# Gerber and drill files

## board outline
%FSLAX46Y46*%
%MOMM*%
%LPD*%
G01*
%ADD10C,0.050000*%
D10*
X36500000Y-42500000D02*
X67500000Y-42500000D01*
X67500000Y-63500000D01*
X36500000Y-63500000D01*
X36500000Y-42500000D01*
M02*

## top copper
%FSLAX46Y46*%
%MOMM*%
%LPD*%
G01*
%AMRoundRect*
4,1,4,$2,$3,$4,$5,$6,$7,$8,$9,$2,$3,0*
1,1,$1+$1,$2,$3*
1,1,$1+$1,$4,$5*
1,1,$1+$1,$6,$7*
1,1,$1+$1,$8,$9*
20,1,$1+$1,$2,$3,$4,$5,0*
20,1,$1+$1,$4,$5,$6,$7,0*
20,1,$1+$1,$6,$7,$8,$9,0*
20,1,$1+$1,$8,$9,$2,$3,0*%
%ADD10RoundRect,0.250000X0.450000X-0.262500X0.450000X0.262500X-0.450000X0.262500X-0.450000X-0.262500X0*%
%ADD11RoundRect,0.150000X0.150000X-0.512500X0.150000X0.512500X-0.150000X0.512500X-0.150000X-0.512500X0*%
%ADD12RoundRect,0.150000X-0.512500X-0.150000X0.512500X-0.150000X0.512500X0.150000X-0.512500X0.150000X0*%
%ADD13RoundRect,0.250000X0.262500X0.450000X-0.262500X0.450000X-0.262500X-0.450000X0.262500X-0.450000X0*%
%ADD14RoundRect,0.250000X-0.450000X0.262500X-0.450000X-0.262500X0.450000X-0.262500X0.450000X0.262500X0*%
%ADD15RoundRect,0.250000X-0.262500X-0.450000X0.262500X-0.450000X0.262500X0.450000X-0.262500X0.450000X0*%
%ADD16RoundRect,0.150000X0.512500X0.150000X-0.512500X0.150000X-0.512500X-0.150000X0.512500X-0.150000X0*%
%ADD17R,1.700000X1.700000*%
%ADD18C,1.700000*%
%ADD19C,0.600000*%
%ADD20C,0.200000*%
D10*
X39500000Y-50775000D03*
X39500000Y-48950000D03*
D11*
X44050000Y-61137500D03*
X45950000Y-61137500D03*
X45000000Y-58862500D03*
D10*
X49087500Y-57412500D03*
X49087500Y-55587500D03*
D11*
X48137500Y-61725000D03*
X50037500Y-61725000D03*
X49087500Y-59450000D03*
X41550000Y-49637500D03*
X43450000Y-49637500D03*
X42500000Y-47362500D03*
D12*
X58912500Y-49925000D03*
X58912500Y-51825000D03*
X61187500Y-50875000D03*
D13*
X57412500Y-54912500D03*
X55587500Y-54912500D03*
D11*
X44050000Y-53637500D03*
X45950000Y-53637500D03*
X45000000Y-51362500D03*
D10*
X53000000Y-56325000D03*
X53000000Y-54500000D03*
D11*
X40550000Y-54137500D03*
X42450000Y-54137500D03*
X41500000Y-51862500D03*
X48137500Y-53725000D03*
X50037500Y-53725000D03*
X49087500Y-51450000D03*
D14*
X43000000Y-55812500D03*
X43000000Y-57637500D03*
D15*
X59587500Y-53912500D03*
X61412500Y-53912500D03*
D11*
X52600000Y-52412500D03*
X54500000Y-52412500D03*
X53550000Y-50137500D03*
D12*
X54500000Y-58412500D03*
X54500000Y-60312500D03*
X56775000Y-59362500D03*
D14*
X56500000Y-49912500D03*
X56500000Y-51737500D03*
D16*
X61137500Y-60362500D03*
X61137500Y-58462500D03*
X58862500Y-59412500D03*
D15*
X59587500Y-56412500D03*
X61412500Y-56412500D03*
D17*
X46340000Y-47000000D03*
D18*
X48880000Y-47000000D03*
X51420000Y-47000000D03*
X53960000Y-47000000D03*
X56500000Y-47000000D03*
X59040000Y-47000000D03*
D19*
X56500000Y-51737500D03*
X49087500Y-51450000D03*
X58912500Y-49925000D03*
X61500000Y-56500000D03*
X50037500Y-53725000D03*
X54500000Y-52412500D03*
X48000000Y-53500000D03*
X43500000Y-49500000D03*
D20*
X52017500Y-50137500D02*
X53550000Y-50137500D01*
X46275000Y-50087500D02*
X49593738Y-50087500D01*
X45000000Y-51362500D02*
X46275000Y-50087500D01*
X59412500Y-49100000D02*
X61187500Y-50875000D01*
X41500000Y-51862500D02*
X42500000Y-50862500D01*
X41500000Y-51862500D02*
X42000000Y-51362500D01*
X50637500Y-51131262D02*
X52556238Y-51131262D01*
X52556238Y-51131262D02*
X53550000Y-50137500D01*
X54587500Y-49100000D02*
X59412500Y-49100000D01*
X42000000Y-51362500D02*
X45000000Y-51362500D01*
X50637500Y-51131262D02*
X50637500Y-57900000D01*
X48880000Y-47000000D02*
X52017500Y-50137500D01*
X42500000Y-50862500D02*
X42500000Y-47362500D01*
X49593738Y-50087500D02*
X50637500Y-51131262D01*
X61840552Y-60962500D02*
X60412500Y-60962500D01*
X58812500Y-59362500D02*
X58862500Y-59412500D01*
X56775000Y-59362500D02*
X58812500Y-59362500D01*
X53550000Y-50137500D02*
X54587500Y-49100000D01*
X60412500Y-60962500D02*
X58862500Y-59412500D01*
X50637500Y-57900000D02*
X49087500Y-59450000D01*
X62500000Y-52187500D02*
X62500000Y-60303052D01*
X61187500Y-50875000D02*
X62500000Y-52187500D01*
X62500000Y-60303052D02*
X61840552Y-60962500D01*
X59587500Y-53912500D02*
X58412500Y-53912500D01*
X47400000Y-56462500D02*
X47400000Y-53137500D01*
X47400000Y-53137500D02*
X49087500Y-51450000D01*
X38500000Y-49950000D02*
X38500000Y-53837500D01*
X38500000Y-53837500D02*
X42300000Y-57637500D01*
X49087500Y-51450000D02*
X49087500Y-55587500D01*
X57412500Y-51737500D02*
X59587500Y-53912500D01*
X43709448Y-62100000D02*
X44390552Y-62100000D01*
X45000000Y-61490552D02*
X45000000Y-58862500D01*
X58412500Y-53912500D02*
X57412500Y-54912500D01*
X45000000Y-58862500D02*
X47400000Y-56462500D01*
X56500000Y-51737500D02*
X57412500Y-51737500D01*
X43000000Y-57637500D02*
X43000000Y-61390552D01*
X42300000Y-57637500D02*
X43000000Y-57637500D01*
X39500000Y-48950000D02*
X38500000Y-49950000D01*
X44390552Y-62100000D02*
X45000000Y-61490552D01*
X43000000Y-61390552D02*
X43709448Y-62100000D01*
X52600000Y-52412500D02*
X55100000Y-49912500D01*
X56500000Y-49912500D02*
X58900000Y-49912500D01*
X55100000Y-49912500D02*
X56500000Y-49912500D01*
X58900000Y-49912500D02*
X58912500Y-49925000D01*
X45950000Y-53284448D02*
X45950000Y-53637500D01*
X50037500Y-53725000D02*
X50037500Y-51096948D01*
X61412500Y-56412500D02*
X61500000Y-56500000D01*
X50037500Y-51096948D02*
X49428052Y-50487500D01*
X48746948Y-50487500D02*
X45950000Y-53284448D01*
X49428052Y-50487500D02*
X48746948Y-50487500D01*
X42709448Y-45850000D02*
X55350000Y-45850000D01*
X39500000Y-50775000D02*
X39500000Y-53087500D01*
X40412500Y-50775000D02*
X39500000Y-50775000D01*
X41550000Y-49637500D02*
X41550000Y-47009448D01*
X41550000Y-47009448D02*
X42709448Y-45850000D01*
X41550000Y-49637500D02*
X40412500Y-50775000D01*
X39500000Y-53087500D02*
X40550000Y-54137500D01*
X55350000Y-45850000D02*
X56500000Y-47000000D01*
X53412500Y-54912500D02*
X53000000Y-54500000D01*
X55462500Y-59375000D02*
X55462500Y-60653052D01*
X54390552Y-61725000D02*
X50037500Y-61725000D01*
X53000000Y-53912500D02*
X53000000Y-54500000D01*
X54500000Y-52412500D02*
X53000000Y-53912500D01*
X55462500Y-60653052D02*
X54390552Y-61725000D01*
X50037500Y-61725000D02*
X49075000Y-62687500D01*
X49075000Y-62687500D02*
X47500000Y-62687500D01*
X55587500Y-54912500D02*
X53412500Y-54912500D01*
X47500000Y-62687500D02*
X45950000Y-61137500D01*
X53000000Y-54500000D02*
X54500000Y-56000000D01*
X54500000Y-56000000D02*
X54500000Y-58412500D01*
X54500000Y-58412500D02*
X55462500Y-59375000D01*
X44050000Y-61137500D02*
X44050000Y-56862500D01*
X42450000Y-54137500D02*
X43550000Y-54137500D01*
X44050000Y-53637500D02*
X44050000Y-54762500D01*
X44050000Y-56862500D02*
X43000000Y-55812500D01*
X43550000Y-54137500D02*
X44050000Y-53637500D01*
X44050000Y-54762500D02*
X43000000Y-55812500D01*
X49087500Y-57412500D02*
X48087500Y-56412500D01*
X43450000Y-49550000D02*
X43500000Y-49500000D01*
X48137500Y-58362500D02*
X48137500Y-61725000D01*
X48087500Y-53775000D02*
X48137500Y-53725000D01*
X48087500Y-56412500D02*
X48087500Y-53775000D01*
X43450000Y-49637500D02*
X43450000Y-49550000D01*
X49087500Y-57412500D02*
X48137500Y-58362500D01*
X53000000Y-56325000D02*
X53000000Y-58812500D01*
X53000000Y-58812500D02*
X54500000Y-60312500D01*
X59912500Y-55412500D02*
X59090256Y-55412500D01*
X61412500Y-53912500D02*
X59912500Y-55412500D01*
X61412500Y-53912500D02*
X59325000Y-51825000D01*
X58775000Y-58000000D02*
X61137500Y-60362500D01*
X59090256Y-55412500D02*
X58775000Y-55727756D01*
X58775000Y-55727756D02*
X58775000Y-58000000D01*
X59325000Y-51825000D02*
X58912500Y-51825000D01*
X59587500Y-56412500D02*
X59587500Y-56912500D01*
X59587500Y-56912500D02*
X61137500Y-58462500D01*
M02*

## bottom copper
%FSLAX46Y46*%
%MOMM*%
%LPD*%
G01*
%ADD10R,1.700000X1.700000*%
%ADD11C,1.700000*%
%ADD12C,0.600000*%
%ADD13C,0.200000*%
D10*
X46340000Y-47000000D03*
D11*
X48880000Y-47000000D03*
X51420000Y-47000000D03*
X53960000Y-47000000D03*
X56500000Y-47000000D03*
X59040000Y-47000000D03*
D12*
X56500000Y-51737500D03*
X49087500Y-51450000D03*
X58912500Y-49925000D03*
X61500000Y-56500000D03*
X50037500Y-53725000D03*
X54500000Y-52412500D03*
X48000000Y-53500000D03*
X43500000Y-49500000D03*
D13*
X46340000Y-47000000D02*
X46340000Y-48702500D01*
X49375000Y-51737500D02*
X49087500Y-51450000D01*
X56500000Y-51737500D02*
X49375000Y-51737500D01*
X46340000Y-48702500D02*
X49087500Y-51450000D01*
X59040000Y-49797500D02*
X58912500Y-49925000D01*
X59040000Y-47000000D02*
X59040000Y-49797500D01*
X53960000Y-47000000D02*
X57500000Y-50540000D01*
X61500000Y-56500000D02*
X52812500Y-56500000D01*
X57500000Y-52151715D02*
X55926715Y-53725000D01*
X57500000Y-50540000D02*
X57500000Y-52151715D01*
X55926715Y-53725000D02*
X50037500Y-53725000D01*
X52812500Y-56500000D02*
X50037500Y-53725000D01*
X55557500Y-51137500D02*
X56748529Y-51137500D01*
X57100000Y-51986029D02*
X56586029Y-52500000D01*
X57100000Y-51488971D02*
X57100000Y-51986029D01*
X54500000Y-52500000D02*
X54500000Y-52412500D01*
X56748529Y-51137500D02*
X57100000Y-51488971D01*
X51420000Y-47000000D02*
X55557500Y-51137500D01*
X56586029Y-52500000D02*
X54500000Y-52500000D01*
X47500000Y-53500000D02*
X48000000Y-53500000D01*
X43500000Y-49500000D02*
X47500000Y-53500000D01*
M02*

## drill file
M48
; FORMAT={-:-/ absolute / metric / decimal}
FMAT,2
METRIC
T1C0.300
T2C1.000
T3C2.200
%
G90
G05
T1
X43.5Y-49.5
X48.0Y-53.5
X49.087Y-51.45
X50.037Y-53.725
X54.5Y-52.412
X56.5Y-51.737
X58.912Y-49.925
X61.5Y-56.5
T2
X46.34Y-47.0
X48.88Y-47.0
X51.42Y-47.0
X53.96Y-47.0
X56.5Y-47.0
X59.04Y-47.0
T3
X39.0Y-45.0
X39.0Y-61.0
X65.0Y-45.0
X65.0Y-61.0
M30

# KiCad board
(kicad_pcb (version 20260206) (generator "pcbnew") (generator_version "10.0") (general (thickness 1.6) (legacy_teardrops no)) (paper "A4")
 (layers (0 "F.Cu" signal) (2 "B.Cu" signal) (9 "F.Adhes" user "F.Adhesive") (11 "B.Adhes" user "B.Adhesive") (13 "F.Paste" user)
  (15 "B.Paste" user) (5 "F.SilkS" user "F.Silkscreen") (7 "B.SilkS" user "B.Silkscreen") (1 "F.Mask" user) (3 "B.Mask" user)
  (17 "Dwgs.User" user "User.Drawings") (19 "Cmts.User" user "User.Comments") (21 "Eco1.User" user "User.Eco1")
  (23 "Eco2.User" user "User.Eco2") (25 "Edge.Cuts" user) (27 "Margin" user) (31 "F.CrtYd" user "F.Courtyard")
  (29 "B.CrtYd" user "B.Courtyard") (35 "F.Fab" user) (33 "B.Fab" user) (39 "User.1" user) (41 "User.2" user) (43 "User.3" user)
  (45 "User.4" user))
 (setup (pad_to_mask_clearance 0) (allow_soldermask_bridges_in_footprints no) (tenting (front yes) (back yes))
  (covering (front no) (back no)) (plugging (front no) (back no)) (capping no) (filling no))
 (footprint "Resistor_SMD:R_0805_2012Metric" (layer "F.Cu") (at 39.5 49.8625 90)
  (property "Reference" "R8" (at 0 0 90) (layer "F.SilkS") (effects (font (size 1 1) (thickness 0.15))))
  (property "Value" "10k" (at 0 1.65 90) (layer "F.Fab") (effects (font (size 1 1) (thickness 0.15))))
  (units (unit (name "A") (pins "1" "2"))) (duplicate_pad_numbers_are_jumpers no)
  (pad "1" smd roundrect (at -0.9125 0 90) (size 1.025 1.4) (layers "F.Cu" "F.Mask" "F.Paste") (roundrect_rratio 0.243902) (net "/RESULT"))
  (pad "2" smd roundrect (at 0.9125 0 90) (size 1.025 1.4) (layers "F.Cu" "F.Mask" "F.Paste") (roundrect_rratio 0.243902) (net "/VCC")))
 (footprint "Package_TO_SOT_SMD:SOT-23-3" (layer "F.Cu") (at 45 60 90)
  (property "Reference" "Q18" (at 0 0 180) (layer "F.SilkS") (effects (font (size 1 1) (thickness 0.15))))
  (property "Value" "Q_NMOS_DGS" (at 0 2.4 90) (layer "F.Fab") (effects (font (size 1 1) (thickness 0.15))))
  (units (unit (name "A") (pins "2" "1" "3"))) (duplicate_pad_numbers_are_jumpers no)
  (pad "1" smd roundrect (at -1.1375 -0.95 90) (size 1.325 0.6) (layers "F.Cu" "F.Mask" "F.Paste") (roundrect_rratio 0.25)
   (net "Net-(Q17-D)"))
  (pad "2" smd roundrect (at -1.1375 0.95 90) (size 1.325 0.6) (layers "F.Cu" "F.Mask" "F.Paste") (roundrect_rratio 0.25) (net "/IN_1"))
  (pad "3" smd roundrect (at 1.1375 0 90) (size 1.325 0.6) (layers "F.Cu" "F.Mask" "F.Paste") (roundrect_rratio 0.25) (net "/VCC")))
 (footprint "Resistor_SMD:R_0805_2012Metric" (layer "F.Cu") (at 49.0875 56.5 90)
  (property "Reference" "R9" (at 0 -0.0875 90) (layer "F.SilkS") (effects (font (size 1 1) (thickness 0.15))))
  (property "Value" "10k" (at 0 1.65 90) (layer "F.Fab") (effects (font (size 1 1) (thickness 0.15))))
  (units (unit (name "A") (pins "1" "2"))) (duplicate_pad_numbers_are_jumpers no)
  (pad "1" smd roundrect (at -0.9125 0 90) (size 1.025 1.4) (layers "F.Cu" "F.Mask" "F.Paste") (roundrect_rratio 0.243902)
   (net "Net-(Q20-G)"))
  (pad "2" smd roundrect (at 0.9125 0 90) (size 1.025 1.4) (layers "F.Cu" "F.Mask" "F.Paste") (roundrect_rratio 0.243902) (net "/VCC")))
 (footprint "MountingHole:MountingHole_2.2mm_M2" (layer "F.Cu") (at 65 45)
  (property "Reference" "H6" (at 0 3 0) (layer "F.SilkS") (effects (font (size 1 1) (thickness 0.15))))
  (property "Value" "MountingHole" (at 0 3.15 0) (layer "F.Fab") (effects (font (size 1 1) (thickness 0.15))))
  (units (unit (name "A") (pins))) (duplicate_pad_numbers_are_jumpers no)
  (pad "" np_thru_hole circle (at 0 0) (size 2.2 2.2) (drill 2.2) (layers "*.Cu" "*.Mask")))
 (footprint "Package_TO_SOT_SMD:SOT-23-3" (layer "F.Cu") (at 49.0875 60.5875 90)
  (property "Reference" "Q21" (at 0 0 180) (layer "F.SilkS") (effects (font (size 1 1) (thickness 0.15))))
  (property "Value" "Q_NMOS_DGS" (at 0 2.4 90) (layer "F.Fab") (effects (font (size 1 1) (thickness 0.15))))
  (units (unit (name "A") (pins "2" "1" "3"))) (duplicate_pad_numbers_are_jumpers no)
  (pad "1" smd roundrect (at -1.1375 -0.95 90) (size 1.325 0.6) (layers "F.Cu" "F.Mask" "F.Paste") (roundrect_rratio 0.25)
   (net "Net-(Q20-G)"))
  (pad "2" smd roundrect (at -1.1375 0.95 90) (size 1.325 0.6) (layers "F.Cu" "F.Mask" "F.Paste") (roundrect_rratio 0.25) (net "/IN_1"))
  (pad "3" smd roundrect (at 1.1375 0 90) (size 1.325 0.6) (layers "F.Cu" "F.Mask" "F.Paste") (roundrect_rratio 0.25) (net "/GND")))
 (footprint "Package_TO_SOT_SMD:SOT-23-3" (layer "F.Cu") (at 42.5 48.5 90)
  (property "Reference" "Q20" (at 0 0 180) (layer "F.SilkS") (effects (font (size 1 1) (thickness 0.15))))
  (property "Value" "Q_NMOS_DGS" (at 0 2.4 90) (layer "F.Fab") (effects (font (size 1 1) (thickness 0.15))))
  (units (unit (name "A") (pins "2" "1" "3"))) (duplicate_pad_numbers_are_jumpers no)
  (pad "1" smd roundrect (at -1.1375 -0.95 90) (size 1.325 0.6) (layers "F.Cu" "F.Mask" "F.Paste") (roundrect_rratio 0.25) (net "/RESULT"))
  (pad "2" smd roundrect (at -1.1375 0.95 90) (size 1.325 0.6) (layers "F.Cu" "F.Mask" "F.Paste") (roundrect_rratio 0.25)
   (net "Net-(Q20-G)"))
  (pad "3" smd roundrect (at 1.1375 0 90) (size 1.325 0.6) (layers "F.Cu" "F.Mask" "F.Paste") (roundrect_rratio 0.25) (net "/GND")))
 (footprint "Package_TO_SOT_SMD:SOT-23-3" (layer "F.Cu") (at 60.05 50.875)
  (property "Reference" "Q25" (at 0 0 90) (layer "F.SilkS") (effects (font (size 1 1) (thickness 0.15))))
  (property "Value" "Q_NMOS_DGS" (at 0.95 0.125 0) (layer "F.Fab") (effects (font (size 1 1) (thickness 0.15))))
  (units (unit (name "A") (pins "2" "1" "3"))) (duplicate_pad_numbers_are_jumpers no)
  (pad "1" smd roundrect (at -1.1375 -0.95) (size 1.325 0.6) (layers "F.Cu" "F.Mask" "F.Paste") (roundrect_rratio 0.25) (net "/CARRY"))
  (pad "2" smd roundrect (at -1.1375 0.95) (size 1.325 0.6) (layers "F.Cu" "F.Mask" "F.Paste") (roundrect_rratio 0.25) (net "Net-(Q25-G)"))
  (pad "3" smd roundrect (at 1.1375 0) (size 1.325 0.6) (layers "F.Cu" "F.Mask" "F.Paste") (roundrect_rratio 0.25) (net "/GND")))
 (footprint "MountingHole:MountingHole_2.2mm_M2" (layer "F.Cu") (at 39 45)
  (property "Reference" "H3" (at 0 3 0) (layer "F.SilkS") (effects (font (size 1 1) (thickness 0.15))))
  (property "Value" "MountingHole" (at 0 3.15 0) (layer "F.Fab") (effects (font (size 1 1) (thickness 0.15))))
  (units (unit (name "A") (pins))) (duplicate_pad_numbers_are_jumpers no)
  (pad "" np_thru_hole circle (at 0 0) (size 2.2 2.2) (drill 2.2) (layers "*.Cu" "*.Mask")))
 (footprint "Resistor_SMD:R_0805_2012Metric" (layer "F.Cu") (at 56.5 54.9125 180)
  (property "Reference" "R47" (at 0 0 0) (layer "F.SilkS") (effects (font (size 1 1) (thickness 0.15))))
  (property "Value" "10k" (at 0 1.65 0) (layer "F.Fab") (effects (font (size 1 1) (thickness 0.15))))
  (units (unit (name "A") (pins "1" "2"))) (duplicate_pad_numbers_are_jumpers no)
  (pad "1" smd roundrect (at -0.9125 0 180) (size 1.025 1.4) (layers "F.Cu" "F.Mask" "F.Paste") (roundrect_rratio 0.243902) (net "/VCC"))
  (pad "2" smd roundrect (at 0.9125 0 180) (size 1.025 1.4) (layers "F.Cu" "F.Mask" "F.Paste") (roundrect_rratio 0.243902) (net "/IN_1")))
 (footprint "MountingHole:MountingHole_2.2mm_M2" (layer "F.Cu") (at 39 61)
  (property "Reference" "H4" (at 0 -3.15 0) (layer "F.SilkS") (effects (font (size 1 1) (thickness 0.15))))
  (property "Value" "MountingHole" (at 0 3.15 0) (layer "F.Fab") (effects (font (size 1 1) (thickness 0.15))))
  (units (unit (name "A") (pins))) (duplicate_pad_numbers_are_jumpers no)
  (pad "" np_thru_hole circle (at 0 0) (size 2.2 2.2) (drill 2.2) (layers "*.Cu" "*.Mask")))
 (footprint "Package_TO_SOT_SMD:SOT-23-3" (layer "F.Cu") (at 45 52.5 90)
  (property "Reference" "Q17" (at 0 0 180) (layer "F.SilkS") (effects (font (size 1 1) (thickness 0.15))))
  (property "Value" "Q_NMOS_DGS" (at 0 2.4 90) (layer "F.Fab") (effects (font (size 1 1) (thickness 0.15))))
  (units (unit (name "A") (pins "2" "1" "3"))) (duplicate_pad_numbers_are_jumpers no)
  (pad "1" smd roundrect (at -1.1375 -0.95 90) (size 1.325 0.6) (layers "F.Cu" "F.Mask" "F.Paste") (roundrect_rratio 0.25)
   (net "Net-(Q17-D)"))
  (pad "2" smd roundrect (at -1.1375 0.95 90) (size 1.325 0.6) (layers "F.Cu" "F.Mask" "F.Paste") (roundrect_rratio 0.25) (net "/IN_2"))
  (pad "3" smd roundrect (at 1.1375 0 90) (size 1.325 0.6) (layers "F.Cu" "F.Mask" "F.Paste") (roundrect_rratio 0.25) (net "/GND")))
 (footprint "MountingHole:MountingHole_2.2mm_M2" (layer "F.Cu") (at 65 61)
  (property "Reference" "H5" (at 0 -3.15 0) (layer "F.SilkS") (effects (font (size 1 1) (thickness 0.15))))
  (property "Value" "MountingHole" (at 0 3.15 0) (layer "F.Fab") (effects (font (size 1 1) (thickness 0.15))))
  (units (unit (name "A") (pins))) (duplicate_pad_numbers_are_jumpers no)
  (pad "" np_thru_hole circle (at 0 0) (size 2.2 2.2) (drill 2.2) (layers "*.Cu" "*.Mask")))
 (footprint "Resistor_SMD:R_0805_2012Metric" (layer "F.Cu") (at 53 55.4125 90)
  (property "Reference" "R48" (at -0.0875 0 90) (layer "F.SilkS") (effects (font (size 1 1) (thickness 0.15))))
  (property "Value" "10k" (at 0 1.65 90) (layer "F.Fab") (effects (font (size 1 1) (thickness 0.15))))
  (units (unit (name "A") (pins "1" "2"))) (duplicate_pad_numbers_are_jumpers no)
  (pad "1" smd roundrect (at -0.9125 0 90) (size 1.025 1.4) (layers "F.Cu" "F.Mask" "F.Paste") (roundrect_rratio 0.243902)
   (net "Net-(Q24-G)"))
  (pad "2" smd roundrect (at 0.9125 0 90) (size 1.025 1.4) (layers "F.Cu" "F.Mask" "F.Paste") (roundrect_rratio 0.243902) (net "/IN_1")))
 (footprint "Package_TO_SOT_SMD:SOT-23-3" (layer "F.Cu") (at 41.5 53 90)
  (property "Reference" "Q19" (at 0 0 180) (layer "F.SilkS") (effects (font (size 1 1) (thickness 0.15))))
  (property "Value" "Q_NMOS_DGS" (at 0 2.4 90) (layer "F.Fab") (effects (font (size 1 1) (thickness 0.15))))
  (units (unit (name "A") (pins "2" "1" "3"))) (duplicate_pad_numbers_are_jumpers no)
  (pad "1" smd roundrect (at -1.1375 -0.95 90) (size 1.325 0.6) (layers "F.Cu" "F.Mask" "F.Paste") (roundrect_rratio 0.25) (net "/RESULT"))
  (pad "2" smd roundrect (at -1.1375 0.95 90) (size 1.325 0.6) (layers "F.Cu" "F.Mask" "F.Paste") (roundrect_rratio 0.25)
   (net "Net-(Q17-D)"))
  (pad "3" smd roundrect (at 1.1375 0 90) (size 1.325 0.6) (layers "F.Cu" "F.Mask" "F.Paste") (roundrect_rratio 0.25) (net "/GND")))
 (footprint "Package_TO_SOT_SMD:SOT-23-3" (layer "F.Cu") (at 49.0875 52.5875 90)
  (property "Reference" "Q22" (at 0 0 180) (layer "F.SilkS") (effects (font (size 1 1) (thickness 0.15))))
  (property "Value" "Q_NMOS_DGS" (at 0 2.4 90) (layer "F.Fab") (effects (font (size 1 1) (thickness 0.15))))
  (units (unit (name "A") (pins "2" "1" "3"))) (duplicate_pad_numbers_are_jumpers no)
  (pad "1" smd roundrect (at -1.1375 -0.95 90) (size 1.325 0.6) (layers "F.Cu" "F.Mask" "F.Paste") (roundrect_rratio 0.25)
   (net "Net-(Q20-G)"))
  (pad "2" smd roundrect (at -1.1375 0.95 90) (size 1.325 0.6) (layers "F.Cu" "F.Mask" "F.Paste") (roundrect_rratio 0.25) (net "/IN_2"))
  (pad "3" smd roundrect (at 1.1375 0 90) (size 1.325 0.6) (layers "F.Cu" "F.Mask" "F.Paste") (roundrect_rratio 0.25) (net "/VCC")))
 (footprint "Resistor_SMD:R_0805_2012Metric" (layer "F.Cu") (at 43 56.725 -90)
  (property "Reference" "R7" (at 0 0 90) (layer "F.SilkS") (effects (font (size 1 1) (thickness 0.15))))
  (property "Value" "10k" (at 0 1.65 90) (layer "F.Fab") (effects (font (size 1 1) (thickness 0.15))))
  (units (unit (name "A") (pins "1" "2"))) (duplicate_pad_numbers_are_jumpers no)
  (pad "1" smd roundrect (at -0.9125 0 270) (size 1.025 1.4) (layers "F.Cu" "F.Mask" "F.Paste") (roundrect_rratio 0.243902)
   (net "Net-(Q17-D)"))
  (pad "2" smd roundrect (at 0.9125 0 270) (size 1.025 1.4) (layers "F.Cu" "F.Mask" "F.Paste") (roundrect_rratio 0.243902) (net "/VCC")))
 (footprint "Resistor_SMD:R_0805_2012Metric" (layer "F.Cu") (at 60.5 53.9125)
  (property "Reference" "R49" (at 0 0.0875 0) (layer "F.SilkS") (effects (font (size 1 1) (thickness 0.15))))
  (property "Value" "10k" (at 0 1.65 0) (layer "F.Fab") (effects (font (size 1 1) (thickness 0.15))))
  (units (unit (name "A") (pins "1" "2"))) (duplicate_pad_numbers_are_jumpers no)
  (pad "1" smd roundrect (at -0.9125 0) (size 1.025 1.4) (layers "F.Cu" "F.Mask" "F.Paste") (roundrect_rratio 0.243902) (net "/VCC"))
  (pad "2" smd roundrect (at 0.9125 0) (size 1.025 1.4) (layers "F.Cu" "F.Mask" "F.Paste") (roundrect_rratio 0.243902) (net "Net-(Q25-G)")))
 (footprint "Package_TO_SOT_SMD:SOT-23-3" (layer "F.Cu") (at 53.55 51.275 90)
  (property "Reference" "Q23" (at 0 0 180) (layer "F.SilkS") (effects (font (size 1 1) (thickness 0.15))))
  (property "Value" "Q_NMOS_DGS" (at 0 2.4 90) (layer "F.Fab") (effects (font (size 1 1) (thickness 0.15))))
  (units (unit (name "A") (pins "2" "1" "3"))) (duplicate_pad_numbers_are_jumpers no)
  (pad "1" smd roundrect (at -1.1375 -0.95 90) (size 1.325 0.6) (layers "F.Cu" "F.Mask" "F.Paste") (roundrect_rratio 0.25) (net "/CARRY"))
  (pad "2" smd roundrect (at -1.1375 0.95 90) (size 1.325 0.6) (layers "F.Cu" "F.Mask" "F.Paste") (roundrect_rratio 0.25) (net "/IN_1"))
  (pad "3" smd roundrect (at 1.1375 0 90) (size 1.325 0.6) (layers "F.Cu" "F.Mask" "F.Paste") (roundrect_rratio 0.25) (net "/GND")))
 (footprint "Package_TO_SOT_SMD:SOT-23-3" (layer "F.Cu") (at 55.6375 59.3625)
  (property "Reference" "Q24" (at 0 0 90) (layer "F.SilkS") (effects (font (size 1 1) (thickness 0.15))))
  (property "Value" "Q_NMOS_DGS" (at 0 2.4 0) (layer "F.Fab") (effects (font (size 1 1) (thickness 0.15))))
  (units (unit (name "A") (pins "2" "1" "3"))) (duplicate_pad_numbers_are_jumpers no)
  (pad "1" smd roundrect (at -1.1375 -0.95) (size 1.325 0.6) (layers "F.Cu" "F.Mask" "F.Paste") (roundrect_rratio 0.25) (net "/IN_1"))
  (pad "2" smd roundrect (at -1.1375 0.95) (size 1.325 0.6) (layers "F.Cu" "F.Mask" "F.Paste") (roundrect_rratio 0.25) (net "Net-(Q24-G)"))
  (pad "3" smd roundrect (at 1.1375 0) (size 1.325 0.6) (layers "F.Cu" "F.Mask" "F.Paste") (roundrect_rratio 0.25) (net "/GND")))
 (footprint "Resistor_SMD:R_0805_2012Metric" (layer "F.Cu") (at 56.5 50.825 -90)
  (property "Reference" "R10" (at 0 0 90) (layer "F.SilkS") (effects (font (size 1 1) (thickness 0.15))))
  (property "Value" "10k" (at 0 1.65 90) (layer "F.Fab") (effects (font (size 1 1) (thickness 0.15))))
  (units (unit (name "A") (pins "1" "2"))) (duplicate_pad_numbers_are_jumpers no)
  (pad "1" smd roundrect (at -0.9125 0 270) (size 1.025 1.4) (layers "F.Cu" "F.Mask" "F.Paste") (roundrect_rratio 0.243902) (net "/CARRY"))
  (pad "2" smd roundrect (at 0.9125 0 270) (size 1.025 1.4) (layers "F.Cu" "F.Mask" "F.Paste") (roundrect_rratio 0.243902) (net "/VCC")))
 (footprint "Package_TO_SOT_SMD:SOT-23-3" (layer "F.Cu") (at 60 59.4125 180)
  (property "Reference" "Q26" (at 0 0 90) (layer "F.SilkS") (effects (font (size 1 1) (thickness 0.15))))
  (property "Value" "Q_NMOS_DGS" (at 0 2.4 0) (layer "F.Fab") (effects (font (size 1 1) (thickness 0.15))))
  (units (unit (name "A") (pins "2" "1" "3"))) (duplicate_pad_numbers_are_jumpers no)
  (pad "1" smd roundrect (at -1.1375 -0.95 180) (size 1.325 0.6) (layers "F.Cu" "F.Mask" "F.Paste") (roundrect_rratio 0.25)
   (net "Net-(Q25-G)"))
  (pad "2" smd roundrect (at -1.1375 0.95 180) (size 1.325 0.6) (layers "F.Cu" "F.Mask" "F.Paste") (roundrect_rratio 0.25)
   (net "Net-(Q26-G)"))
  (pad "3" smd roundrect (at 1.1375 0 180) (size 1.325 0.6) (layers "F.Cu" "F.Mask" "F.Paste") (roundrect_rratio 0.25) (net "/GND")))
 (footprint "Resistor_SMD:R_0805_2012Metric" (layer "F.Cu") (at 60.5 56.4125)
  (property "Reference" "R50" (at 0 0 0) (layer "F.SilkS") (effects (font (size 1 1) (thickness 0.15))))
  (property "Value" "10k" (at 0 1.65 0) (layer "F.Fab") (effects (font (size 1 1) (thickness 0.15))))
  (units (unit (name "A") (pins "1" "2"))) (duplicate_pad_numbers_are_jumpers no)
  (pad "1" smd roundrect (at -0.9125 0) (size 1.025 1.4) (layers "F.Cu" "F.Mask" "F.Paste") (roundrect_rratio 0.243902) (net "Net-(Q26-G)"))
  (pad "2" smd roundrect (at 0.9125 0) (size 1.025 1.4) (layers "F.Cu" "F.Mask" "F.Paste") (roundrect_rratio 0.243902) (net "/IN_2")))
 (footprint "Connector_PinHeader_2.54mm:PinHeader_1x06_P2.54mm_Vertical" (layer "F.Cu") (at 46.34 47 90)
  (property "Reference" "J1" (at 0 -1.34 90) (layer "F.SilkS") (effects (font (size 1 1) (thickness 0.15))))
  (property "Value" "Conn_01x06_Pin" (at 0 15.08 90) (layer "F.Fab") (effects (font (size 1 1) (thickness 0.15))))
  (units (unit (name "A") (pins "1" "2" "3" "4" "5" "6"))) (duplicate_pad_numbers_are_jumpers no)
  (pad "1" thru_hole rect (at 0 0 90) (size 1.7 1.7) (drill 1) (layers "*.Cu" "*.Mask") (remove_unused_layers no) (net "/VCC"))
  (pad "2" thru_hole circle (at 0 2.54 90) (size 1.7 1.7) (drill 1) (layers "*.Cu" "*.Mask") (remove_unused_layers no) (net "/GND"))
  (pad "3" thru_hole circle (at 0 5.08 90) (size 1.7 1.7) (drill 1) (layers "*.Cu" "*.Mask") (remove_unused_layers no) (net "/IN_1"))
  (pad "4" thru_hole circle (at 0 7.62 90) (size 1.7 1.7) (drill 1) (layers "*.Cu" "*.Mask") (remove_unused_layers no) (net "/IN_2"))
  (pad "5" thru_hole circle (at 0 10.16 90) (size 1.7 1.7) (drill 1) (layers "*.Cu" "*.Mask") (remove_unused_layers no) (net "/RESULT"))
  (pad "6" thru_hole circle (at 0 12.7 90) (size 1.7 1.7) (drill 1) (layers "*.Cu" "*.Mask") (remove_unused_layers no) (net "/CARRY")))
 (gr_rect (start 36.5 42.5) (end 67.5 63.5) (stroke (width 0.05) (type default)) (fill no) (layer "Edge.Cuts"))
 (segment (start 52.0175 50.1375) (end 53.55 50.1375) (width 0.2) (layer "F.Cu") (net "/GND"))
 (segment (start 46.275 50.0875) (end 49.593738 50.0875) (width 0.2) (layer "F.Cu") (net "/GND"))
 (segment (start 45 51.3625) (end 46.275 50.0875) (width 0.2) (layer "F.Cu") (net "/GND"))
 (segment (start 59.4125 49.1) (end 61.1875 50.875) (width 0.2) (layer "F.Cu") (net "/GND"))
 (segment (start 41.5 51.8625) (end 42.5 50.8625) (width 0.2) (layer "F.Cu") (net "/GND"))
 (segment (start 41.5 51.8625) (end 42 51.3625) (width 0.2) (layer "F.Cu") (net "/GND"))
 (segment (start 50.6375 51.131262) (end 52.556238 51.131262) (width 0.2) (layer "F.Cu") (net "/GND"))
 (segment (start 52.556238 51.131262) (end 53.55 50.1375) (width 0.2) (layer "F.Cu") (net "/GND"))
 (segment (start 54.5875 49.1) (end 59.4125 49.1) (width 0.2) (layer "F.Cu") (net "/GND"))
 (segment (start 42 51.3625) (end 45 51.3625) (width 0.2) (layer "F.Cu") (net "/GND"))
 (segment (start 50.6375 51.131262) (end 50.6375 57.9) (width 0.2) (layer "F.Cu") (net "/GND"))
 (segment (start 48.88 47) (end 52.0175 50.1375) (width 0.2) (layer "F.Cu") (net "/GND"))
 (segment (start 42.5 50.8625) (end 42.5 47.3625) (width 0.2) (layer "F.Cu") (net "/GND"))
 (segment (start 49.593738 50.0875) (end 50.6375 51.131262) (width 0.2) (layer "F.Cu") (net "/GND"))
 (segment (start 61.840552 60.9625) (end 60.4125 60.9625) (width 0.2) (layer "F.Cu") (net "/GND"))
 (segment (start 58.8125 59.3625) (end 58.8625 59.4125) (width 0.2) (layer "F.Cu") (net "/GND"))
 (segment (start 56.775 59.3625) (end 58.8125 59.3625) (width 0.2) (layer "F.Cu") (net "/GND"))
 (segment (start 53.55 50.1375) (end 54.5875 49.1) (width 0.2) (layer "F.Cu") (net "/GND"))
 (segment (start 60.4125 60.9625) (end 58.8625 59.4125) (width 0.2) (layer "F.Cu") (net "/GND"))
 (segment (start 50.6375 57.9) (end 49.0875 59.45) (width 0.2) (layer "F.Cu") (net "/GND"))
 (segment (start 62.5 52.1875) (end 62.5 60.303052) (width 0.2) (layer "F.Cu") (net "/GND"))
 (segment (start 61.1875 50.875) (end 62.5 52.1875) (width 0.2) (layer "F.Cu") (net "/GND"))
 (segment (start 62.5 60.303052) (end 61.840552 60.9625) (width 0.2) (layer "F.Cu") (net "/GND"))
 (segment (start 59.5875 53.9125) (end 58.4125 53.9125) (width 0.2) (layer "F.Cu") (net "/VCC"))
 (segment (start 47.4 56.4625) (end 47.4 53.1375) (width 0.2) (layer "F.Cu") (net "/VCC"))
 (segment (start 47.4 53.1375) (end 49.0875 51.45) (width 0.2) (layer "F.Cu") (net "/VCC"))
 (segment (start 38.5 49.95) (end 38.5 53.8375) (width 0.2) (layer "F.Cu") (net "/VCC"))
 (segment (start 38.5 53.8375) (end 42.3 57.6375) (width 0.2) (layer "F.Cu") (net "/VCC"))
 (segment (start 49.0875 51.45) (end 49.0875 55.5875) (width 0.2) (layer "F.Cu") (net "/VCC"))
 (segment (start 57.4125 51.7375) (end 59.5875 53.9125) (width 0.2) (layer "F.Cu") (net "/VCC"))
 (segment (start 43.709448 62.1) (end 44.390552 62.1) (width 0.2) (layer "F.Cu") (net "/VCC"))
 (segment (start 45 61.490552) (end 45 58.8625) (width 0.2) (layer "F.Cu") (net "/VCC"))
 (segment (start 58.4125 53.9125) (end 57.4125 54.9125) (width 0.2) (layer "F.Cu") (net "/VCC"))
 (segment (start 45 58.8625) (end 47.4 56.4625) (width 0.2) (layer "F.Cu") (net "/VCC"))
 (segment (start 56.5 51.7375) (end 57.4125 51.7375) (width 0.2) (layer "F.Cu") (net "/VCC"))
 (segment (start 43 57.6375) (end 43 61.390552) (width 0.2) (layer "F.Cu") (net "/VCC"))
 (segment (start 42.3 57.6375) (end 43 57.6375) (width 0.2) (layer "F.Cu") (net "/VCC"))
 (segment (start 39.5 48.95) (end 38.5 49.95) (width 0.2) (layer "F.Cu") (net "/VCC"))
 (segment (start 44.390552 62.1) (end 45 61.490552) (width 0.2) (layer "F.Cu") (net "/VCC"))
 (segment (start 43 61.390552) (end 43.709448 62.1) (width 0.2) (layer "F.Cu") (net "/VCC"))
 (via (at 56.5 51.7375) (size 0.6) (drill 0.3) (layers "F.Cu" "B.Cu") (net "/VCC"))
 (via (at 49.0875 51.45) (size 0.6) (drill 0.3) (layers "F.Cu" "B.Cu") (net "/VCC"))
 (segment (start 46.34 47) (end 46.34 48.7025) (width 0.2) (layer "B.Cu") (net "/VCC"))
 (segment (start 49.375 51.7375) (end 49.0875 51.45) (width 0.2) (layer "B.Cu") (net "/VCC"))
 (segment (start 56.5 51.7375) (end 49.375 51.7375) (width 0.2) (layer "B.Cu") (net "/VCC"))
 (segment (start 46.34 48.7025) (end 49.0875 51.45) (width 0.2) (layer "B.Cu") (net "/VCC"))
 (segment (start 52.6 52.4125) (end 55.1 49.9125) (width 0.2) (layer "F.Cu") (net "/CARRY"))
 (segment (start 56.5 49.9125) (end 58.9 49.9125) (width 0.2) (layer "F.Cu") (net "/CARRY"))
 (segment (start 55.1 49.9125) (end 56.5 49.9125) (width 0.2) (layer "F.Cu") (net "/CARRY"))
 (segment (start 58.9 49.9125) (end 58.9125 49.925) (width 0.2) (layer "F.Cu") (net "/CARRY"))
 (via (at 58.9125 49.925) (size 0.6) (drill 0.3) (layers "F.Cu" "B.Cu") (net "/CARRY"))
 (segment (start 59.04 49.7975) (end 58.9125 49.925) (width 0.2) (layer "B.Cu") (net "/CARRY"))
 (segment (start 59.04 47) (end 59.04 49.7975) (width 0.2) (layer "B.Cu") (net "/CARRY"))
 (segment (start 45.95 53.284448) (end 45.95 53.6375) (width 0.2) (layer "F.Cu") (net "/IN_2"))
 (segment (start 50.0375 53.725) (end 50.0375 51.096948) (width 0.2) (layer "F.Cu") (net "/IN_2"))
 (segment (start 61.4125 56.4125) (end 61.5 56.5) (width 0.2) (layer "F.Cu") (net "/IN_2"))
 (segment (start 50.0375 51.096948) (end 49.428052 50.4875) (width 0.2) (layer "F.Cu") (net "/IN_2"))
 (segment (start 48.746948 50.4875) (end 45.95 53.284448) (width 0.2) (layer "F.Cu") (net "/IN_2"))
 (segment (start 49.428052 50.4875) (end 48.746948 50.4875) (width 0.2) (layer "F.Cu") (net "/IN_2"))
 (via (at 61.5 56.5) (size 0.6) (drill 0.3) (layers "F.Cu" "B.Cu") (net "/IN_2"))
 (via (at 50.0375 53.725) (size 0.6) (drill 0.3) (layers "F.Cu" "B.Cu") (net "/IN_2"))
 (segment (start 53.96 47) (end 57.5 50.54) (width 0.2) (layer "B.Cu") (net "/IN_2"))
 (segment (start 61.5 56.5) (end 52.8125 56.5) (width 0.2) (layer "B.Cu") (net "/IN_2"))
 (segment (start 57.5 52.151715) (end 55.926715 53.725) (width 0.2) (layer "B.Cu") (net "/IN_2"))
 (segment (start 57.5 50.54) (end 57.5 52.151715) (width 0.2) (layer "B.Cu") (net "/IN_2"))
 (segment (start 55.926715 53.725) (end 50.0375 53.725) (width 0.2) (layer "B.Cu") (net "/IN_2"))
 (segment (start 52.8125 56.5) (end 50.0375 53.725) (width 0.2) (layer "B.Cu") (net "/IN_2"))
 (segment (start 42.709448 45.85) (end 55.35 45.85) (width 0.2) (layer "F.Cu") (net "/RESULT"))
 (segment (start 39.5 50.775) (end 39.5 53.0875) (width 0.2) (layer "F.Cu") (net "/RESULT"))
 (segment (start 40.4125 50.775) (end 39.5 50.775) (width 0.2) (layer "F.Cu") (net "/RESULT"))
 (segment (start 41.55 49.6375) (end 41.55 47.009448) (width 0.2) (layer "F.Cu") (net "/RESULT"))
 (segment (start 41.55 47.009448) (end 42.709448 45.85) (width 0.2) (layer "F.Cu") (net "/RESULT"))
 (segment (start 41.55 49.6375) (end 40.4125 50.775) (width 0.2) (layer "F.Cu") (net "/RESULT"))
 (segment (start 39.5 53.0875) (end 40.55 54.1375) (width 0.2) (layer "F.Cu") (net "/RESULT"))
 (segment (start 55.35 45.85) (end 56.5 47) (width 0.2) (layer "F.Cu") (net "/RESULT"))
 (segment (start 53.4125 54.9125) (end 53 54.5) (width 0.2) (layer "F.Cu") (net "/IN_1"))
 (segment (start 55.4625 59.375) (end 55.4625 60.653052) (width 0.2) (layer "F.Cu") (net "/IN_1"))
 (segment (start 54.390552 61.725) (end 50.0375 61.725) (width 0.2) (layer "F.Cu") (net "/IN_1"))
 (segment (start 53 53.9125) (end 53 54.5) (width 0.2) (layer "F.Cu") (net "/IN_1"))
 (segment (start 54.5 52.4125) (end 53 53.9125) (width 0.2) (layer "F.Cu") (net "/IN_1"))
 (segment (start 55.4625 60.653052) (end 54.390552 61.725) (width 0.2) (layer "F.Cu") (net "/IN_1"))
 (segment (start 50.0375 61.725) (end 49.075 62.6875) (width 0.2) (layer "F.Cu") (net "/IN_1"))
 (segment (start 49.075 62.6875) (end 47.5 62.6875) (width 0.2) (layer "F.Cu") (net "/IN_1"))
 (segment (start 55.5875 54.9125) (end 53.4125 54.9125) (width 0.2) (layer "F.Cu") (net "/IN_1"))
 (segment (start 47.5 62.6875) (end 45.95 61.1375) (width 0.2) (layer "F.Cu") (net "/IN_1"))
 (segment (start 53 54.5) (end 54.5 56) (width 0.2) (layer "F.Cu") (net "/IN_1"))
 (segment (start 54.5 56) (end 54.5 58.4125) (width 0.2) (layer "F.Cu") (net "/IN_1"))
 (segment (start 54.5 58.4125) (end 55.4625 59.375) (width 0.2) (layer "F.Cu") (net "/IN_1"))
 (via (at 54.5 52.4125) (size 0.6) (drill 0.3) (layers "F.Cu" "B.Cu") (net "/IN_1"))
 (segment (start 55.5575 51.1375) (end 56.748529 51.1375) (width 0.2) (layer "B.Cu") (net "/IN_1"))
 (segment (start 57.1 51.986029) (end 56.586029 52.5) (width 0.2) (layer "B.Cu") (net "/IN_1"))
 (segment (start 57.1 51.488971) (end 57.1 51.986029) (width 0.2) (layer "B.Cu") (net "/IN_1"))
 (segment (start 54.5 52.5) (end 54.5 52.4125) (width 0.2) (layer "B.Cu") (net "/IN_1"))
 (segment (start 56.748529 51.1375) (end 57.1 51.488971) (width 0.2) (layer "B.Cu") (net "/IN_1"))
 (segment (start 51.42 47) (end 55.5575 51.1375) (width 0.2) (layer "B.Cu") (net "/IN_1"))
 (segment (start 56.586029 52.5) (end 54.5 52.5) (width 0.2) (layer "B.Cu") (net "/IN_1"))
 (segment (start 44.05 61.1375) (end 44.05 56.8625) (width 0.2) (layer "F.Cu") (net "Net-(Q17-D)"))
 (segment (start 42.45 54.1375) (end 43.55 54.1375) (width 0.2) (layer "F.Cu") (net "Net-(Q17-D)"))
 (segment (start 44.05 53.6375) (end 44.05 54.7625) (width 0.2) (layer "F.Cu") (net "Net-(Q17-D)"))
 (segment (start 44.05 56.8625) (end 43 55.8125) (width 0.2) (layer "F.Cu") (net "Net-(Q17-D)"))
 (segment (start 43.55 54.1375) (end 44.05 53.6375) (width 0.2) (layer "F.Cu") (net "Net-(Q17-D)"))
 (segment (start 44.05 54.7625) (end 43 55.8125) (width 0.2) (layer "F.Cu") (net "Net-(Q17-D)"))
 (segment (start 49.0875 57.4125) (end 48.0875 56.4125) (width 0.2) (layer "F.Cu") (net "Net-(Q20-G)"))
 (segment (start 43.45 49.55) (end 43.5 49.5) (width 0.2) (layer "F.Cu") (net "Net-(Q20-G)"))
 (segment (start 48.1375 58.3625) (end 48.1375 61.725) (width 0.2) (layer "F.Cu") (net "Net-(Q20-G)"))
 (segment (start 48.0875 53.775) (end 48.1375 53.725) (width 0.2) (layer "F.Cu") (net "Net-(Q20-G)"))
 (segment (start 48.0875 56.4125) (end 48.0875 53.775) (width 0.2) (layer "F.Cu") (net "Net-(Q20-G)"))
 (segment (start 43.45 49.6375) (end 43.45 49.55) (width 0.2) (layer "F.Cu") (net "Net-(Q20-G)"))
 (segment (start 49.0875 57.4125) (end 48.1375 58.3625) (width 0.2) (layer "F.Cu") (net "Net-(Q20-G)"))
 (via (at 48 53.5) (size 0.6) (drill 0.3) (layers "F.Cu" "B.Cu") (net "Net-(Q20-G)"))
 (via (at 43.5 49.5) (size 0.6) (drill 0.3) (layers "F.Cu" "B.Cu") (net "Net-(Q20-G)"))
 (segment (start 47.5 53.5) (end 48 53.5) (width 0.2) (layer "B.Cu") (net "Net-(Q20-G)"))
 (segment (start 43.5 49.5) (end 47.5 53.5) (width 0.2) (layer "B.Cu") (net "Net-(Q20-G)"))
 (segment (start 53 56.325) (end 53 58.8125) (width 0.2) (layer "F.Cu") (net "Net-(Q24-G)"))
 (segment (start 53 58.8125) (end 54.5 60.3125) (width 0.2) (layer "F.Cu") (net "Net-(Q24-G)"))
 (segment (start 59.9125 55.4125) (end 59.090256 55.4125) (width 0.2) (layer "F.Cu") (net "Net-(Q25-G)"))
 (segment (start 61.4125 53.9125) (end 59.9125 55.4125) (width 0.2) (layer "F.Cu") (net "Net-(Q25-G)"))
 (segment (start 61.4125 53.9125) (end 59.325 51.825) (width 0.2) (layer "F.Cu") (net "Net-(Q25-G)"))
 (segment (start 58.775 58) (end 61.1375 60.3625) (width 0.2) (layer "F.Cu") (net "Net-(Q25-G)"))
 (segment (start 59.090256 55.4125) (end 58.775 55.727756) (width 0.2) (layer "F.Cu") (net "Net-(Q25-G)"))
 (segment (start 58.775 55.727756) (end 58.775 58) (width 0.2) (layer "F.Cu") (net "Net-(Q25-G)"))
 (segment (start 59.325 51.825) (end 58.9125 51.825) (width 0.2) (layer "F.Cu") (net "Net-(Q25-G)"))
 (segment (start 59.5875 56.4125) (end 59.5875 56.9125) (width 0.2) (layer "F.Cu") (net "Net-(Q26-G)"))
 (segment (start 59.5875 56.9125) (end 61.1375 58.4625) (width 0.2) (layer "F.Cu") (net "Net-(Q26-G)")))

